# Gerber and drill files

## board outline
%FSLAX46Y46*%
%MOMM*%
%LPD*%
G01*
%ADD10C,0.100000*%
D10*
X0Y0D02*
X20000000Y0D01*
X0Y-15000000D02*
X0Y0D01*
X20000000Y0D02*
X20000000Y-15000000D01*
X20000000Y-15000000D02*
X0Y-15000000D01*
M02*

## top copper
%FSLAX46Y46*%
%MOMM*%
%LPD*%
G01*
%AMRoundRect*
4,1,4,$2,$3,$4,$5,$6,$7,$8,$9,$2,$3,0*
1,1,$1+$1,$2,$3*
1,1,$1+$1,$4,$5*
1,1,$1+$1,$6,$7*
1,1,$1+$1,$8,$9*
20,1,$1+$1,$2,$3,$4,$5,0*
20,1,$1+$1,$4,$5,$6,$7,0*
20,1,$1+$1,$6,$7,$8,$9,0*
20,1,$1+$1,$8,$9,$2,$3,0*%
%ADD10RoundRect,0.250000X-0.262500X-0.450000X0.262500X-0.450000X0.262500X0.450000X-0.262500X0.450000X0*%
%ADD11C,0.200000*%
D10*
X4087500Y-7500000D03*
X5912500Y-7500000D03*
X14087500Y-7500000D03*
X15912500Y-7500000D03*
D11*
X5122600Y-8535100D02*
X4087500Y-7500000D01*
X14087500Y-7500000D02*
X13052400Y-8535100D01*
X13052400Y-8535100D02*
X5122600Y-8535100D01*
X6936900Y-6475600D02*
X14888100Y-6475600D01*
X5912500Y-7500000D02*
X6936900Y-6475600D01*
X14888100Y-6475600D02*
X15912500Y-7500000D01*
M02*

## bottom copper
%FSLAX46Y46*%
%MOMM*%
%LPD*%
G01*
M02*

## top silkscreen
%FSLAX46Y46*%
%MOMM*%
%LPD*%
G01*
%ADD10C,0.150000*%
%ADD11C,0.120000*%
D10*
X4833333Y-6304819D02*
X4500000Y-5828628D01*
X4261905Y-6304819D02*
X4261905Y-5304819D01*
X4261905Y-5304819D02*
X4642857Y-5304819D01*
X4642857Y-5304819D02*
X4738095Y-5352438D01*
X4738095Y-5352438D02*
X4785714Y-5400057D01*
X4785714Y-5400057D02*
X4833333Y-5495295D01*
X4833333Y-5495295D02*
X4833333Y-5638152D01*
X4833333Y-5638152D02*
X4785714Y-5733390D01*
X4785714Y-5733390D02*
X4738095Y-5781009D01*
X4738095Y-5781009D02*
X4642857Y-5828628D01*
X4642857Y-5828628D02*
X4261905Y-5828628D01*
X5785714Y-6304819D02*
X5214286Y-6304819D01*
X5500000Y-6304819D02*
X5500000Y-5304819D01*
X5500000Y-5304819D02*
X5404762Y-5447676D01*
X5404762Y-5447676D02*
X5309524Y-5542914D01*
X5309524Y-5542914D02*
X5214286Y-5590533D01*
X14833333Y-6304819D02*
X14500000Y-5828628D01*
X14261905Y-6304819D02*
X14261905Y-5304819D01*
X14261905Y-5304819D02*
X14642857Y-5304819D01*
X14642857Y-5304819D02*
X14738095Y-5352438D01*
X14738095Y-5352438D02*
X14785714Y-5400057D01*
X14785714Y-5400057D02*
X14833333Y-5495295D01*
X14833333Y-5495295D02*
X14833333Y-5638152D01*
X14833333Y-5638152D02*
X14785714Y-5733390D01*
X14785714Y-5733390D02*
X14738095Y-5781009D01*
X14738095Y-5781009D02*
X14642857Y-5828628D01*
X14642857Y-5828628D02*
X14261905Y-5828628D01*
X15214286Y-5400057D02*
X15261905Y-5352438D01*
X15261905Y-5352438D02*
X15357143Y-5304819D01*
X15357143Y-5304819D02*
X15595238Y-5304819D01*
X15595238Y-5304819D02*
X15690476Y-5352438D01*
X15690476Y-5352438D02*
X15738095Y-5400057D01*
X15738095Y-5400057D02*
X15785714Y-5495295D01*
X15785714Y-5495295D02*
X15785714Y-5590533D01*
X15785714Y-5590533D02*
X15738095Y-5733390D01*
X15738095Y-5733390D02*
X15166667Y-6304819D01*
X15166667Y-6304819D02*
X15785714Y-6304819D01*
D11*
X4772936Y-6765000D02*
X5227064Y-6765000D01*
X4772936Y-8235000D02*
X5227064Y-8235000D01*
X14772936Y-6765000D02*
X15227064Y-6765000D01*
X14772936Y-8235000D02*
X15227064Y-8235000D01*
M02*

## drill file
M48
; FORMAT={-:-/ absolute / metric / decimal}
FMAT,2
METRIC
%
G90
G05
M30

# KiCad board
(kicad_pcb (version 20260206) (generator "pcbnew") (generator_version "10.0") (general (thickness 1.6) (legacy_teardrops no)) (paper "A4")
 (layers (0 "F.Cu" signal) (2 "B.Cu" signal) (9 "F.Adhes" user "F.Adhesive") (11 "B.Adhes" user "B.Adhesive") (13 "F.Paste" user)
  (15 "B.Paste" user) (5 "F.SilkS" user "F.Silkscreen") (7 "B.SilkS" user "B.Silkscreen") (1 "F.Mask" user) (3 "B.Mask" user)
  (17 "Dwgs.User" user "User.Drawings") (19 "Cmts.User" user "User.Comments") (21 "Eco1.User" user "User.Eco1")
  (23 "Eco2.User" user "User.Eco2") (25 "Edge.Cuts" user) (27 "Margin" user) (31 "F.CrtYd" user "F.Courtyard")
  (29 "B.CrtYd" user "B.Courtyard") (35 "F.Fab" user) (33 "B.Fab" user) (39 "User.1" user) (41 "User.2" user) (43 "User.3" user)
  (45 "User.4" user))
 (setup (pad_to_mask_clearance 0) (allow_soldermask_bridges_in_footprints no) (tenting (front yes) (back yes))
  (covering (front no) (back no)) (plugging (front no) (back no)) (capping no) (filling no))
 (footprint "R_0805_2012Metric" (layer "F.Cu") (at 5 7.5)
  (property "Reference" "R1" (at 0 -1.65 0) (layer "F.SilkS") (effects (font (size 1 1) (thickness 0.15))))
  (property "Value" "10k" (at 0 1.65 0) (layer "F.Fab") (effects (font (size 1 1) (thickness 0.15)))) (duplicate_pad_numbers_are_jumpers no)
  (fp_line (start -0.227064 -0.735) (end 0.227064 -0.735) (stroke (width 0.12) (type solid)) (layer "F.SilkS"))
  (fp_line (start -0.227064 0.735) (end 0.227064 0.735) (stroke (width 0.12) (type solid)) (layer "F.SilkS"))
  (pad "1" smd roundrect (at -0.9125 0) (size 1.025 1.4) (layers "F.Cu" "F.Mask" "F.Paste") (roundrect_rratio 0.243902) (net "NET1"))
  (pad "2" smd roundrect (at 0.9125 0) (size 1.025 1.4) (layers "F.Cu" "F.Mask" "F.Paste") (roundrect_rratio 0.243902) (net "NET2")))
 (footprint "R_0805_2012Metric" (layer "F.Cu") (at 15 7.5)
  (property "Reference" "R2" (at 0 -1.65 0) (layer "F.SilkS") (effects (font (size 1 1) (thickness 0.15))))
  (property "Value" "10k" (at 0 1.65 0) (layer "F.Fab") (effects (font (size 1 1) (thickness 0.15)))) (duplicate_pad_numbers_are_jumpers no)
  (fp_line (start -0.227064 -0.735) (end 0.227064 -0.735) (stroke (width 0.12) (type solid)) (layer "F.SilkS"))
  (fp_line (start -0.227064 0.735) (end 0.227064 0.735) (stroke (width 0.12) (type solid)) (layer "F.SilkS"))
  (pad "1" smd roundrect (at -0.9125 0) (size 1.025 1.4) (layers "F.Cu" "F.Mask" "F.Paste") (roundrect_rratio 0.243902) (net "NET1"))
  (pad "2" smd roundrect (at 0.9125 0) (size 1.025 1.4) (layers "F.Cu" "F.Mask" "F.Paste") (roundrect_rratio 0.243902) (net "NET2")))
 (gr_line (start 0 0) (end 20 0) (stroke (width 0.1) (type default)) (layer "Edge.Cuts"))
 (gr_line (start 0 15) (end 0 0) (stroke (width 0.1) (type default)) (layer "Edge.Cuts"))
 (gr_line (start 20 0) (end 20 15) (stroke (width 0.1) (type default)) (layer "Edge.Cuts"))
 (gr_line (start 20 15) (end 0 15) (stroke (width 0.1) (type default)) (layer "Edge.Cuts"))
 (segment (start 5.1226 8.5351) (end 4.0875 7.5) (width 0.2) (layer "F.Cu") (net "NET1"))
 (segment (start 14.0875 7.5) (end 13.0524 8.5351) (width 0.2) (layer "F.Cu") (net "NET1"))
 (segment (start 13.0524 8.5351) (end 5.1226 8.5351) (width 0.2) (layer "F.Cu") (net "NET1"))
 (segment (start 6.9369 6.4756) (end 14.8881 6.4756) (width 0.2) (layer "F.Cu") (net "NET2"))
 (segment (start 5.9125 7.5) (end 6.9369 6.4756) (width 0.2) (layer "F.Cu") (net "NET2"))
 (segment (start 14.8881 6.4756) (end 15.9125 7.5) (width 0.2) (layer "F.Cu") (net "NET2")))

